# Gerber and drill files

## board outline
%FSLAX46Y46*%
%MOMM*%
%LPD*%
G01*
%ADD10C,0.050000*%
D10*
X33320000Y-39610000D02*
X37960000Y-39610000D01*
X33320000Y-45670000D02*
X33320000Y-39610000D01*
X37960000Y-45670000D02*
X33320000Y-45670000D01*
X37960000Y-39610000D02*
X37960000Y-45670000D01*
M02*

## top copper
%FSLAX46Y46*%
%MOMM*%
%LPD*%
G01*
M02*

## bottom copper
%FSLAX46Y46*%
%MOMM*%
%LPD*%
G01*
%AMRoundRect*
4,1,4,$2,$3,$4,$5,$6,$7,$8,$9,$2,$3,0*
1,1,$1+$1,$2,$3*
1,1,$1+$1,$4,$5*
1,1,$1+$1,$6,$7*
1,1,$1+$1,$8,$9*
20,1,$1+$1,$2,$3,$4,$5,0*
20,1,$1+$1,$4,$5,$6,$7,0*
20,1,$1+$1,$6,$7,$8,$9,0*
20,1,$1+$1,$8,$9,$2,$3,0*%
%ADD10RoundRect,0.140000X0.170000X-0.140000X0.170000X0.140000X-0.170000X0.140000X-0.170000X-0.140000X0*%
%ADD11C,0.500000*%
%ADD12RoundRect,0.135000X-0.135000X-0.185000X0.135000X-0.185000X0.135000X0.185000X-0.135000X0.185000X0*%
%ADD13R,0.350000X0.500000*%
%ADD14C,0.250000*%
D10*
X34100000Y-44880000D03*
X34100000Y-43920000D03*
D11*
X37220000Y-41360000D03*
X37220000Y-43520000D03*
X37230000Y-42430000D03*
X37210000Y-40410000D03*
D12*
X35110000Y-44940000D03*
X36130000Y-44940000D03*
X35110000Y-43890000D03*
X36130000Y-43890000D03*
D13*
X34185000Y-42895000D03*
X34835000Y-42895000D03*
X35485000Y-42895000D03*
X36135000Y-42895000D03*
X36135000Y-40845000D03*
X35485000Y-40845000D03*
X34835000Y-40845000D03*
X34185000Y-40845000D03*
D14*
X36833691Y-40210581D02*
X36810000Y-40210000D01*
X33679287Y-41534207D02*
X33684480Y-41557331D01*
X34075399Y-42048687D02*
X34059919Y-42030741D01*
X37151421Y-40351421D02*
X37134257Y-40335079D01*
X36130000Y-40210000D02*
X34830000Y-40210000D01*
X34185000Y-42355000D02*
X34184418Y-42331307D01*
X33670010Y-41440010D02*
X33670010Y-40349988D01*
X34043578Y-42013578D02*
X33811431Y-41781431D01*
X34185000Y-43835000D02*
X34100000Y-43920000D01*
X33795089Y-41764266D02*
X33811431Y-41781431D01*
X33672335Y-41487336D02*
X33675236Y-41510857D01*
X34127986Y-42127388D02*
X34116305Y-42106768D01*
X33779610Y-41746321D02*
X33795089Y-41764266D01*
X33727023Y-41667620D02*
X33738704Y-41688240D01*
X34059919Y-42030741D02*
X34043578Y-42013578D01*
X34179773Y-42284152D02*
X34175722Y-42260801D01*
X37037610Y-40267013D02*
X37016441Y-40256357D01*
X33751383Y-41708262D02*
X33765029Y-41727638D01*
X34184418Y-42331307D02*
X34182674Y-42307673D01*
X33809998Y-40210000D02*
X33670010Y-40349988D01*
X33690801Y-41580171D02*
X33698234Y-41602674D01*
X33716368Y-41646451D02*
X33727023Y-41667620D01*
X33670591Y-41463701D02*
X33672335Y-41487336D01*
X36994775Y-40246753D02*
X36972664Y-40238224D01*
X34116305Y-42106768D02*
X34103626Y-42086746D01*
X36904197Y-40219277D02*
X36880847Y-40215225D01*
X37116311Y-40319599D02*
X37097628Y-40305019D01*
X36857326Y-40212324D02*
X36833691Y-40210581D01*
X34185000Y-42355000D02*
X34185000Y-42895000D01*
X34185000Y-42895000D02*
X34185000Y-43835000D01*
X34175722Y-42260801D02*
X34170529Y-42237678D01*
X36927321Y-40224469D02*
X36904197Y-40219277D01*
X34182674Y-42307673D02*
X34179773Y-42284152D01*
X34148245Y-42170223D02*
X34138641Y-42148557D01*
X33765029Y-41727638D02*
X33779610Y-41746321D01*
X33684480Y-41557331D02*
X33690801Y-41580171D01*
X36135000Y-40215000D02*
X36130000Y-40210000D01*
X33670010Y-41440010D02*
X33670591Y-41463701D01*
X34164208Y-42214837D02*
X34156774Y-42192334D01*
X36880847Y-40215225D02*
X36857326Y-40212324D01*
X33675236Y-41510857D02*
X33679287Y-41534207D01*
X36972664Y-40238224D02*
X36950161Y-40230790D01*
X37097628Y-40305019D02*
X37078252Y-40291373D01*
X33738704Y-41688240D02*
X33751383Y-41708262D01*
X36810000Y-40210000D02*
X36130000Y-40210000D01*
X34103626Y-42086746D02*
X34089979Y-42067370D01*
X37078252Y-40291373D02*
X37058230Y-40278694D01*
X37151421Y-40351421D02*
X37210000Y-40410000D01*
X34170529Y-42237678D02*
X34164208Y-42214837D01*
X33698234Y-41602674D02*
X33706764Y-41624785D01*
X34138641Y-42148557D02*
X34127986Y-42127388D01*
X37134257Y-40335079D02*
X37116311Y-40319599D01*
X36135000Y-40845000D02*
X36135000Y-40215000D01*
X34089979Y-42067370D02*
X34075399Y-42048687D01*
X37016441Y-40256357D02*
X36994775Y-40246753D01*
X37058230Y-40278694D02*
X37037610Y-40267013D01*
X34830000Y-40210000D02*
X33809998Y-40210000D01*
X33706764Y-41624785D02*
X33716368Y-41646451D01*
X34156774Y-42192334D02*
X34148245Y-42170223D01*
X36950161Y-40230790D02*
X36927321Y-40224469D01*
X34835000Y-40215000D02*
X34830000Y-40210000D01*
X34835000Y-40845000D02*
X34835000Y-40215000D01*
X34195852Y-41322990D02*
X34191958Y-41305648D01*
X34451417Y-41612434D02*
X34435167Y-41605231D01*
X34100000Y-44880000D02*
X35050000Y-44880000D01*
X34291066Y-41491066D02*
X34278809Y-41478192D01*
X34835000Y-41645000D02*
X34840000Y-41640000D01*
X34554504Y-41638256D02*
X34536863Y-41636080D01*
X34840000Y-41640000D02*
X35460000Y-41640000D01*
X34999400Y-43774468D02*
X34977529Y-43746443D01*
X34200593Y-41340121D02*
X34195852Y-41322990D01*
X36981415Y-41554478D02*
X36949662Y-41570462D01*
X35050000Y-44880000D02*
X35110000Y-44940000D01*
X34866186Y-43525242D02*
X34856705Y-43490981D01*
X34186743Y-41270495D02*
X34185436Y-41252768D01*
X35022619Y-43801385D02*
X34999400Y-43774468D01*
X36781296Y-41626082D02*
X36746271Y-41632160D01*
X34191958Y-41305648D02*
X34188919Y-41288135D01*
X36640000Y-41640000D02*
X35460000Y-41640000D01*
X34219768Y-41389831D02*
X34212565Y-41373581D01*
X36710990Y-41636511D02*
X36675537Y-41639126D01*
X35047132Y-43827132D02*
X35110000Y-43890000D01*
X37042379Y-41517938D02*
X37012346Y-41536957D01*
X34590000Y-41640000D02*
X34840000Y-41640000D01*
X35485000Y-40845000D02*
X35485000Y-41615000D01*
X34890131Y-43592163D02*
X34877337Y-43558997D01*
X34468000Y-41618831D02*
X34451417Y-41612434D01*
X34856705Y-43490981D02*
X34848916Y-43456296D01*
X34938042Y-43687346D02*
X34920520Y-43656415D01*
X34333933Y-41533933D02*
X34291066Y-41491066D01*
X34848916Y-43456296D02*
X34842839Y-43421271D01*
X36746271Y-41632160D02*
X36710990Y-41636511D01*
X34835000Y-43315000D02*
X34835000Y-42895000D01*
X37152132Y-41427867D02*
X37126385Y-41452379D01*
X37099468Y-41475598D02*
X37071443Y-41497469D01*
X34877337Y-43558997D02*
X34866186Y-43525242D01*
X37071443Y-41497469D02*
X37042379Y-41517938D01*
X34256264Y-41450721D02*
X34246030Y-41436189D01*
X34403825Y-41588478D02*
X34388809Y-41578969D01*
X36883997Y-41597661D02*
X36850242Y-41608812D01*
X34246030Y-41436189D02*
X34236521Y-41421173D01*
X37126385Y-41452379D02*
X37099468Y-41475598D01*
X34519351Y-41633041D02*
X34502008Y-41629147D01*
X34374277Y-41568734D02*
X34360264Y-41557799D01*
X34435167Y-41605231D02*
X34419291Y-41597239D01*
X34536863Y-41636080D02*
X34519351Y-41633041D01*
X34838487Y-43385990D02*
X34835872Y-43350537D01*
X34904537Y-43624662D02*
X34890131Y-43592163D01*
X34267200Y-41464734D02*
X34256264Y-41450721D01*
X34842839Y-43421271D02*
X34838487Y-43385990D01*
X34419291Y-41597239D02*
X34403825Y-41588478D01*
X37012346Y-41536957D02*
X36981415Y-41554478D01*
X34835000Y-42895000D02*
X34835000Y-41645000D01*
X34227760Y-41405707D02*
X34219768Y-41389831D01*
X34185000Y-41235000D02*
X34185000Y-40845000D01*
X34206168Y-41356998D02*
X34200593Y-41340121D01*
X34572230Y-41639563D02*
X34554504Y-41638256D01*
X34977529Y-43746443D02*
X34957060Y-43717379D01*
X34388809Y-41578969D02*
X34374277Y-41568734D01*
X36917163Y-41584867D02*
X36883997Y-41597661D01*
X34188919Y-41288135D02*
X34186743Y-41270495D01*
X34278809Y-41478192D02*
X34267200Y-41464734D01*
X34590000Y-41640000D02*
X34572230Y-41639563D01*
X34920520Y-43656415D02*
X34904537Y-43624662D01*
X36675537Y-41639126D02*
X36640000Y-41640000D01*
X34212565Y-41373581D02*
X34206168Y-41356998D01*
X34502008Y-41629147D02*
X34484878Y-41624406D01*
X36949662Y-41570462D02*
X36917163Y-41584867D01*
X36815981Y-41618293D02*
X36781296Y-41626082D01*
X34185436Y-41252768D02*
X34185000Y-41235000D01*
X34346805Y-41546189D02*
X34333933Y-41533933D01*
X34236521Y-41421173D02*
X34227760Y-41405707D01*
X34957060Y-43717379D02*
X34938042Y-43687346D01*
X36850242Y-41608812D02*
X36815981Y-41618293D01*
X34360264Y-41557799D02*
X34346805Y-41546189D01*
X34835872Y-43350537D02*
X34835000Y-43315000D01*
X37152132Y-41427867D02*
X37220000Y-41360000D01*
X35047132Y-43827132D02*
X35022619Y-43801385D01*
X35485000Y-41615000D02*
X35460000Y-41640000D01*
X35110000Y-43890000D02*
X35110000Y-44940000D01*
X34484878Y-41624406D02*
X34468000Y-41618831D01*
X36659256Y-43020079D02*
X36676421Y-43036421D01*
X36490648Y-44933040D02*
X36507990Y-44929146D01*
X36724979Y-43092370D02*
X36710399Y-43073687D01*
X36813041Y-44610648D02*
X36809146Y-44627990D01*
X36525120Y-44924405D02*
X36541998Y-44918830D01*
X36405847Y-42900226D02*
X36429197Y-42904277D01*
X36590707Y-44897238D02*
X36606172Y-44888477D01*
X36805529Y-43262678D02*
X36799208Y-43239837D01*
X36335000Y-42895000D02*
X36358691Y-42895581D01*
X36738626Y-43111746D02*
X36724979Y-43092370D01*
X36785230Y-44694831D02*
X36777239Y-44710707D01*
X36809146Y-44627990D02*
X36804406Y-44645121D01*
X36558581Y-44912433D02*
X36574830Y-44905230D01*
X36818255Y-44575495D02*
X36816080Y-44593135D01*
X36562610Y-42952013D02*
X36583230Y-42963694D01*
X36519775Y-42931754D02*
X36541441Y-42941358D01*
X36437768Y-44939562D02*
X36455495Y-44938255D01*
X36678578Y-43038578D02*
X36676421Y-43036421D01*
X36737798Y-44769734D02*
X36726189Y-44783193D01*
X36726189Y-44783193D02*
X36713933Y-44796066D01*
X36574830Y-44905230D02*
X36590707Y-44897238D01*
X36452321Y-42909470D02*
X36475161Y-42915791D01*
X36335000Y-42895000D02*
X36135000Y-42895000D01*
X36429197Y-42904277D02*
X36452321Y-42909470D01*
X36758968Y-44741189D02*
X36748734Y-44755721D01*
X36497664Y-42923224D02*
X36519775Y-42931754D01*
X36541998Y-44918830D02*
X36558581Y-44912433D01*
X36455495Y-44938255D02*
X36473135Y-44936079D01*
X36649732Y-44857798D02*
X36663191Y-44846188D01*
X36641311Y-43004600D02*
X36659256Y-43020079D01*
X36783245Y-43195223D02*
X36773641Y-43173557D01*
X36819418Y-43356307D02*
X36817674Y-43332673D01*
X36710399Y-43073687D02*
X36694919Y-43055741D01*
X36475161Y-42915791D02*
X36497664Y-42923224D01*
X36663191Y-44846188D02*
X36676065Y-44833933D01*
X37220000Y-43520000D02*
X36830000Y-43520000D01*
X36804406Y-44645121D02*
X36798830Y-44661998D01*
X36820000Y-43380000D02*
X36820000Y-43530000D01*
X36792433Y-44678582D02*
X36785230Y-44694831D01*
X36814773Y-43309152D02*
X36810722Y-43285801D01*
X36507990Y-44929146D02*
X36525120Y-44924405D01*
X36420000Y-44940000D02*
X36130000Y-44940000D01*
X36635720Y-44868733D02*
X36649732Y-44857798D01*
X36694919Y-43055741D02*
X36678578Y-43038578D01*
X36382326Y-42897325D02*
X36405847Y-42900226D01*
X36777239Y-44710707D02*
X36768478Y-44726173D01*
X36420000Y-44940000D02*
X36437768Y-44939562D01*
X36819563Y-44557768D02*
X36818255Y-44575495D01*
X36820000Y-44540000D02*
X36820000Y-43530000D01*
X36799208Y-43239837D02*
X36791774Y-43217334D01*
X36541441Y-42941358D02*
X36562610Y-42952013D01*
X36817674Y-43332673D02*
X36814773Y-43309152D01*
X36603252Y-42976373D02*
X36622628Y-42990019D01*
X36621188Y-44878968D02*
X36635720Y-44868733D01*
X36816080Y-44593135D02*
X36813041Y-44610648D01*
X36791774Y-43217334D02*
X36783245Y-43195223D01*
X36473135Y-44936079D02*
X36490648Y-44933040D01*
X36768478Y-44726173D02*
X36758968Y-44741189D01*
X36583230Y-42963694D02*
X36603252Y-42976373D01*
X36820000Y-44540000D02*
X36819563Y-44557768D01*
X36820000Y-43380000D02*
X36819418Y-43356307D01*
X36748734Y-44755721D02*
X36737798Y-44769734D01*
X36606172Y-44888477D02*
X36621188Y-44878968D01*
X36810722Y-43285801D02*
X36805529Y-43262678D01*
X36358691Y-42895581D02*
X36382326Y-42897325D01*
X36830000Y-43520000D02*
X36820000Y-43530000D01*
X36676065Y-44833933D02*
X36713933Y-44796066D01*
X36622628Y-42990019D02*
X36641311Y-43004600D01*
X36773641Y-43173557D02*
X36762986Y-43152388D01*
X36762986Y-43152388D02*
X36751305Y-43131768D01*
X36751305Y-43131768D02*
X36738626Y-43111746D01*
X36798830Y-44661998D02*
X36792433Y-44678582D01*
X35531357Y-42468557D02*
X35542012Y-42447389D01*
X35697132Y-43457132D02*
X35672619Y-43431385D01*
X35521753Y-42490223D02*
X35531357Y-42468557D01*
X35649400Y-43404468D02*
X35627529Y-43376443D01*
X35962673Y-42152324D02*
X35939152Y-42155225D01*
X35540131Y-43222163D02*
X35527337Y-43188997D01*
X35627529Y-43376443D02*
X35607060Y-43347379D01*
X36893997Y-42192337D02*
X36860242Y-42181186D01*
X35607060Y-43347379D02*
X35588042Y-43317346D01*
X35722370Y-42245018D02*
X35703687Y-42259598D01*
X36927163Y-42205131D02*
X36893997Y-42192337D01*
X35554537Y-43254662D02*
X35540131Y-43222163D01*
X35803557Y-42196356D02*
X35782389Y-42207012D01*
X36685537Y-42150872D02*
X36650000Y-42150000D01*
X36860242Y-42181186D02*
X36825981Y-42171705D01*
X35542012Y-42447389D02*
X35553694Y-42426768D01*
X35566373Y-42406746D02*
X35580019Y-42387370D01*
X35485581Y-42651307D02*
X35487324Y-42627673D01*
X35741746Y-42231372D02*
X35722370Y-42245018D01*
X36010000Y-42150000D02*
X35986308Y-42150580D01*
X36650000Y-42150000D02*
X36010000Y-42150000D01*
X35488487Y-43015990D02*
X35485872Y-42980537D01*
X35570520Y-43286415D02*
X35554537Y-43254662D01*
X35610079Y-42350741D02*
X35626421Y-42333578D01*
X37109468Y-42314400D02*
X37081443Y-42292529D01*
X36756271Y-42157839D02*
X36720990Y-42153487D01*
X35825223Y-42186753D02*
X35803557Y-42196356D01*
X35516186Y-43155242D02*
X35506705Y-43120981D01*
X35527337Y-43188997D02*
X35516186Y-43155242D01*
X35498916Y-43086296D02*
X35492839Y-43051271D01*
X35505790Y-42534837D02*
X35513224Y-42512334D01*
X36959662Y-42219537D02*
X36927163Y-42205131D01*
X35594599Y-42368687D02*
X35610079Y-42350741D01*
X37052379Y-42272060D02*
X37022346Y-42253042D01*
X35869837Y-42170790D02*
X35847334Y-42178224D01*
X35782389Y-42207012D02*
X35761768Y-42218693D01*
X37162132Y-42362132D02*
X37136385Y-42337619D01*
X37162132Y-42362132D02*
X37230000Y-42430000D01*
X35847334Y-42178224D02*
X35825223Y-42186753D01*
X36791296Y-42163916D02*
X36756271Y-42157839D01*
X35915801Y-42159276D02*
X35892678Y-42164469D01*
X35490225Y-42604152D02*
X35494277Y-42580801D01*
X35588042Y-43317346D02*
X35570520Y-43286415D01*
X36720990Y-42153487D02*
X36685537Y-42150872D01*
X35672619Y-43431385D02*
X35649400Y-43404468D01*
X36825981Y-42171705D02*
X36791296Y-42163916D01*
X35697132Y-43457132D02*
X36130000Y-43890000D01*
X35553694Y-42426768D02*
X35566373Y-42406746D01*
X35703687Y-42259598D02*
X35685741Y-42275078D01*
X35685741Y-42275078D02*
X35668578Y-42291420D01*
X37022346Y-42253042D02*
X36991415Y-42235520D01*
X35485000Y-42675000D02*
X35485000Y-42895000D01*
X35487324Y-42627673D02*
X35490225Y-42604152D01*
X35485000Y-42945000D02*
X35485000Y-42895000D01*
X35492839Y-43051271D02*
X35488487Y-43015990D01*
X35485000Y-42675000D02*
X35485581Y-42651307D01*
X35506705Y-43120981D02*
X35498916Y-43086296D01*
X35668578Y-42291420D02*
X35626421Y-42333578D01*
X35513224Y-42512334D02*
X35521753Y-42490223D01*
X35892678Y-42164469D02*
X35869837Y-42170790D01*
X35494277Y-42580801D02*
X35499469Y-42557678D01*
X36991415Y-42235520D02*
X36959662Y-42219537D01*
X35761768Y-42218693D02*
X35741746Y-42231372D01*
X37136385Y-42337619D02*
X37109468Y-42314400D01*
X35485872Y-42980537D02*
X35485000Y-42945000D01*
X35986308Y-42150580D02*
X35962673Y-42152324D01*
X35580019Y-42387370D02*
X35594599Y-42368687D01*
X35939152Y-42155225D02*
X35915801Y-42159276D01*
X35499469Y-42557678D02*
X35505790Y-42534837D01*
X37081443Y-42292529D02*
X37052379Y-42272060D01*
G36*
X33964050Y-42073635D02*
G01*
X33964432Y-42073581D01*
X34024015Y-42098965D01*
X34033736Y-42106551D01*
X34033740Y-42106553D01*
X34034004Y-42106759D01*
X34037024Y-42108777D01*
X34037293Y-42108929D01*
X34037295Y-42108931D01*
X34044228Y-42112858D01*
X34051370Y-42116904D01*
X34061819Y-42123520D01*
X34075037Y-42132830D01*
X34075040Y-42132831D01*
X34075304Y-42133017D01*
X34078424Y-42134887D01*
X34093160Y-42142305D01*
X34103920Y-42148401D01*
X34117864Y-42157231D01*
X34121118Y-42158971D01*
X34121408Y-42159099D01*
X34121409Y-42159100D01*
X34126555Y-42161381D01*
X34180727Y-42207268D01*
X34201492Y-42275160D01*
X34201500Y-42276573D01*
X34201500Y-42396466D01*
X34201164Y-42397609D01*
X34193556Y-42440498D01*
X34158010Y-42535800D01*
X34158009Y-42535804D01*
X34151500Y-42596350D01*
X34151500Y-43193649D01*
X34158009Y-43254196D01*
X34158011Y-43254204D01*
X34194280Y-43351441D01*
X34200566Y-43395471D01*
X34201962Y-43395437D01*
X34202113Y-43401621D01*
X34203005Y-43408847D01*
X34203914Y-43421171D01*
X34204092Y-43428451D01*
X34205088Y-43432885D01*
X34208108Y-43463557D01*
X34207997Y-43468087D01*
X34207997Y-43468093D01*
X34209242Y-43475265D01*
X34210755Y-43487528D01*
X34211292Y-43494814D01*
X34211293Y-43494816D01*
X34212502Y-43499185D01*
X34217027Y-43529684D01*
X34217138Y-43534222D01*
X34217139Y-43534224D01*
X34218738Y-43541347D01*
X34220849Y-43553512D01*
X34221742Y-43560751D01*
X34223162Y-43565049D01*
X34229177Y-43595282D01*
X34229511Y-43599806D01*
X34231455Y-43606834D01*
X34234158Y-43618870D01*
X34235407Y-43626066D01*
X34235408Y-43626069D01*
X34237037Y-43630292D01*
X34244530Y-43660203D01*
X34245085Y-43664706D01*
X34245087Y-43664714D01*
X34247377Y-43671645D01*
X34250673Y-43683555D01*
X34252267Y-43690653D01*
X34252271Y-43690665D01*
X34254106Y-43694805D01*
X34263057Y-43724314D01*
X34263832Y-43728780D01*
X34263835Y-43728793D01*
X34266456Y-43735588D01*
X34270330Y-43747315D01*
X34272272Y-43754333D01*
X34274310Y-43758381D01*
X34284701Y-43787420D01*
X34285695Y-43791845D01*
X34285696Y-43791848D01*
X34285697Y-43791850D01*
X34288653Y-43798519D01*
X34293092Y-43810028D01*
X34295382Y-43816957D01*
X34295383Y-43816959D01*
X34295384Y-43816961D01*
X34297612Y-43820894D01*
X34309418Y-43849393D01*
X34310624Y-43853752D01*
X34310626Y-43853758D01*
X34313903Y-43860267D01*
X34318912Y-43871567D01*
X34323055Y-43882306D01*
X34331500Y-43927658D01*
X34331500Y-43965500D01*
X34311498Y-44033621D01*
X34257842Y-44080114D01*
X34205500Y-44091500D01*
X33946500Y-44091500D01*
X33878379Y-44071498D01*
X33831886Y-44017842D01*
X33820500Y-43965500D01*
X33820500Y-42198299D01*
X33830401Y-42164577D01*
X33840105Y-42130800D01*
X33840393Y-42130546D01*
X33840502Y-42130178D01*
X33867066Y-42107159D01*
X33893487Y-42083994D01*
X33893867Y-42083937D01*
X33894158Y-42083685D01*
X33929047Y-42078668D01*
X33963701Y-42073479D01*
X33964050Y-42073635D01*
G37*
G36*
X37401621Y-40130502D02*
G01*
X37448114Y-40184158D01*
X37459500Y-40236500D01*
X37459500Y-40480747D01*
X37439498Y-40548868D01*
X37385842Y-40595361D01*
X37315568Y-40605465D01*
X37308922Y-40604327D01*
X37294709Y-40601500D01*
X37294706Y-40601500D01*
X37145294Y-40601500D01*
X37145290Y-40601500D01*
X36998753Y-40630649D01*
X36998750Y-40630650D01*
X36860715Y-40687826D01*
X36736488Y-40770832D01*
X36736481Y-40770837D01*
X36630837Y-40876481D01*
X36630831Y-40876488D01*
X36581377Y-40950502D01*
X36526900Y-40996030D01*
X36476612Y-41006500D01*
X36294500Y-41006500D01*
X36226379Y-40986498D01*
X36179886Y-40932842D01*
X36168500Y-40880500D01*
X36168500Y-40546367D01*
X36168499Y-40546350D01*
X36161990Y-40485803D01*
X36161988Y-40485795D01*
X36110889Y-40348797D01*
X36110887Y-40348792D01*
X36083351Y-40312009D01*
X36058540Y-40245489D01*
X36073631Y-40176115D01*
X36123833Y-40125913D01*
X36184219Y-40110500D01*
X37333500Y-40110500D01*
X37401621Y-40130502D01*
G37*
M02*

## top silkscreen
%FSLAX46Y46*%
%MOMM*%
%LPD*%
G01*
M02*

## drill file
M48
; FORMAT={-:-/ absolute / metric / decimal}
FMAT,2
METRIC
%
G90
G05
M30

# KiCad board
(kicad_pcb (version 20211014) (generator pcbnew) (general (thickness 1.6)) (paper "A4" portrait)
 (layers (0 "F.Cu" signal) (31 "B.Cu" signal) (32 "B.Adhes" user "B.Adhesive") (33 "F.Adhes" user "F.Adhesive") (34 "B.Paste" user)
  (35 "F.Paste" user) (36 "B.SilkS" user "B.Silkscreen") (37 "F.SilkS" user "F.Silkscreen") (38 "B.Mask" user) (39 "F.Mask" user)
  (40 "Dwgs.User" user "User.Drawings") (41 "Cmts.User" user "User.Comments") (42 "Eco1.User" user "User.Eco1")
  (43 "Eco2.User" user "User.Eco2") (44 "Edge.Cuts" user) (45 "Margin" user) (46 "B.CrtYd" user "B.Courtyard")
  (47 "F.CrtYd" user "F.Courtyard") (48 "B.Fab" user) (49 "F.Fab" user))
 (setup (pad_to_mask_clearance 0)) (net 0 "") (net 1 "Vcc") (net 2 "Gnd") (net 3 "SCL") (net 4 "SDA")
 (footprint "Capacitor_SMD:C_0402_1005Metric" (layer "B.Cu") (at 34.1 44.4 90)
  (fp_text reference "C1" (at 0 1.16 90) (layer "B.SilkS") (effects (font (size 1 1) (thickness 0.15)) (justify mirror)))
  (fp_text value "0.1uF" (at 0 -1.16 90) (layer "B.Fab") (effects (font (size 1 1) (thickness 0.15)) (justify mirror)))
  (pad "1" smd roundrect locked (at -0.48 0 90) (size 0.56 0.62) (layers "B.Cu" "B.Paste" "B.Mask") (roundrect_rratio 0.25) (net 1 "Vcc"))
  (pad "2" smd roundrect locked (at 0.48 0 90) (size 0.56 0.62) (layers "B.Cu" "B.Paste" "B.Mask") (roundrect_rratio 0.25) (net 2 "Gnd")))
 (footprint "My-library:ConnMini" (layer "B.Cu") (at 37.22 41.36)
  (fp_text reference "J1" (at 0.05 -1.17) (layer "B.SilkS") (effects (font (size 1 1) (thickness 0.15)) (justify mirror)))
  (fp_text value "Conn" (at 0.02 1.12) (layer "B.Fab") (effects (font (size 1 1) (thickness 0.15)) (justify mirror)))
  (pad "1" smd circle locked (at 0 0) (size 0.5 0.5) (layers "B.Cu" "B.Paste" "B.Mask") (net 1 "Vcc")))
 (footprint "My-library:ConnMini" (layer "B.Cu") (at 37.22 43.52)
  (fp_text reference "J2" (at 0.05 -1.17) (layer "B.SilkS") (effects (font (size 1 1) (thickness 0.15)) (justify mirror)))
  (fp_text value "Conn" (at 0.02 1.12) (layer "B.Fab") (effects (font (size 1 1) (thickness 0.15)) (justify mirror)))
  (pad "1" smd circle locked (at 0 0) (size 0.5 0.5) (layers "B.Cu" "B.Paste" "B.Mask") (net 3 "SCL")))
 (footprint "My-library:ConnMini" (layer "B.Cu") (at 37.23 42.43)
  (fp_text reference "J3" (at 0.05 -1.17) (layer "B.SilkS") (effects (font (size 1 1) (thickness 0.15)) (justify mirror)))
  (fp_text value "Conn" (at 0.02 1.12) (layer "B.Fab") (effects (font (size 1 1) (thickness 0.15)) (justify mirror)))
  (pad "1" smd circle locked (at 0 0) (size 0.5 0.5) (layers "B.Cu" "B.Paste" "B.Mask") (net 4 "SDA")))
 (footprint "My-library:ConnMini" (layer "B.Cu") (at 37.21 40.41)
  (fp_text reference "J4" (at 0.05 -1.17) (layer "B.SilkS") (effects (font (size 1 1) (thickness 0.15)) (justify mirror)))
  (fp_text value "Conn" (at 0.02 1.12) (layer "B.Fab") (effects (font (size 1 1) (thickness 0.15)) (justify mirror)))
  (pad "1" smd circle locked (at 0 0) (size 0.5 0.5) (layers "B.Cu" "B.Paste" "B.Mask") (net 2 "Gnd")))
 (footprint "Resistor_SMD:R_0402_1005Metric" (layer "B.Cu") (at 35.62 44.94)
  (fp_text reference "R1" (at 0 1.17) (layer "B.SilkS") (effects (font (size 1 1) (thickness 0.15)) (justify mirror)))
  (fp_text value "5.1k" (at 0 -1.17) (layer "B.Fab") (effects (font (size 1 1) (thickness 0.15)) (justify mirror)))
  (pad "1" smd roundrect locked (at -0.51 0) (size 0.54 0.64) (layers "B.Cu" "B.Paste" "B.Mask") (roundrect_rratio 0.25) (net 1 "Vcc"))
  (pad "2" smd roundrect locked (at 0.51 0) (size 0.54 0.64) (layers "B.Cu" "B.Paste" "B.Mask") (roundrect_rratio 0.25) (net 3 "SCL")))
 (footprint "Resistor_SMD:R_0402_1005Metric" (layer "B.Cu") (at 35.62 43.89)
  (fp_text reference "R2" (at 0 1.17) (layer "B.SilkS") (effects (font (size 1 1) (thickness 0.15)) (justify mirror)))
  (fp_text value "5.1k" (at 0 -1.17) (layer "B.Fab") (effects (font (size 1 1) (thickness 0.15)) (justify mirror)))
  (pad "1" smd roundrect locked (at -0.51 0) (size 0.54 0.64) (layers "B.Cu" "B.Paste" "B.Mask") (roundrect_rratio 0.25) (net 1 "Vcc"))
  (pad "2" smd roundrect locked (at 0.51 0) (size 0.54 0.64) (layers "B.Cu" "B.Paste" "B.Mask") (roundrect_rratio 0.25) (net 4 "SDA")))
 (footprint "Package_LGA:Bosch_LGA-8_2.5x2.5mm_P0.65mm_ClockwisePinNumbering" (layer "B.Cu") (at 35.16 41.87)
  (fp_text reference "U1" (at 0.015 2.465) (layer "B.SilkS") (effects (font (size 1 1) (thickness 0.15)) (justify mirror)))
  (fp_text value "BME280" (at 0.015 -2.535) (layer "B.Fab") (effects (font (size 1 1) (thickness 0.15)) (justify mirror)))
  (pad "1" smd rect locked (at -0.975 1.025 270) (size 0.5 0.35) (layers "B.Cu" "B.Paste" "B.Mask") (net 2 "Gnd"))
  (pad "2" smd rect locked (at -0.325 1.025 270) (size 0.5 0.35) (layers "B.Cu" "B.Paste" "B.Mask") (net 1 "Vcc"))
  (pad "3" smd rect locked (at 0.325 1.025 270) (size 0.5 0.35) (layers "B.Cu" "B.Paste" "B.Mask") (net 4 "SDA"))
  (pad "4" smd rect locked (at 0.975 1.025 270) (size 0.5 0.35) (layers "B.Cu" "B.Paste" "B.Mask") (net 3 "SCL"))
  (pad "5" smd rect locked (at 0.975 -1.025 270) (size 0.5 0.35) (layers "B.Cu" "B.Paste" "B.Mask") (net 2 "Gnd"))
  (pad "6" smd rect locked (at 0.325 -1.025 270) (size 0.5 0.35) (layers "B.Cu" "B.Paste" "B.Mask") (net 1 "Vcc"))
  (pad "7" smd rect locked (at -0.325 -1.025 270) (size 0.5 0.35) (layers "B.Cu" "B.Paste" "B.Mask") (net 2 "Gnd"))
  (pad "8" smd rect locked (at -0.975 -1.025 270) (size 0.5 0.35) (layers "B.Cu" "B.Paste" "B.Mask") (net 1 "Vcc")))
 (gr_line (start 33.32 39.61) (end 37.96 39.61) (layer "Edge.Cuts") (width 0.05))
 (gr_line (start 33.32 45.67) (end 33.32 39.61) (layer "Edge.Cuts") (width 0.05))
 (gr_line (start 37.96 45.67) (end 33.32 45.67) (layer "Edge.Cuts") (width 0.05))
 (gr_line (start 37.96 39.61) (end 37.96 45.67) (layer "Edge.Cuts") (width 0.05))
 (segment (start 36.833691 40.210581) (end 36.81 40.21) (width 0.25) (layer "B.Cu") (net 2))
 (segment (start 33.679287 41.534207) (end 33.68448 41.557331) (width 0.25) (layer "B.Cu") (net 2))
 (segment (start 34.075399 42.048687) (end 34.059919 42.030741) (width 0.25) (layer "B.Cu") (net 2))
 (segment (start 37.151421 40.351421) (end 37.134257 40.335079) (width 0.25) (layer "B.Cu") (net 2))
 (segment (start 36.13 40.21) (end 34.83 40.21) (width 0.25) (layer "B.Cu") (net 2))
 (segment (start 34.185 42.355) (end 34.184418 42.331307) (width 0.25) (layer "B.Cu") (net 2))
 (segment (start 33.67001 41.44001) (end 33.67001 40.349988) (width 0.25) (layer "B.Cu") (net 2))
 (segment (start 34.043578 42.013578) (end 33.811431 41.781431) (width 0.25) (layer "B.Cu") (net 2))
 (segment (start 34.185 43.835) (end 34.1 43.92) (width 0.25) (layer "B.Cu") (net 2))
 (segment (start 33.795089 41.764266) (end 33.811431 41.781431) (width 0.25) (layer "B.Cu") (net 2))
 (segment (start 33.672335 41.487336) (end 33.675236 41.510857) (width 0.25) (layer "B.Cu") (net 2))
 (segment (start 34.127986 42.127388) (end 34.116305 42.106768) (width 0.25) (layer "B.Cu") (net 2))
 (segment (start 33.77961 41.746321) (end 33.795089 41.764266) (width 0.25) (layer "B.Cu") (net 2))
 (segment (start 33.727023 41.66762) (end 33.738704 41.68824) (width 0.25) (layer "B.Cu") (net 2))
 (segment (start 34.059919 42.030741) (end 34.043578 42.013578) (width 0.25) (layer "B.Cu") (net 2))
 (segment (start 34.179773 42.284152) (end 34.175722 42.260801) (width 0.25) (layer "B.Cu") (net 2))
 (segment (start 37.03761 40.267013) (end 37.016441 40.256357) (width 0.25) (layer "B.Cu") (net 2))
 (segment (start 33.751383 41.708262) (end 33.765029 41.727638) (width 0.25) (layer "B.Cu") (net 2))
 (segment (start 34.184418 42.331307) (end 34.182674 42.307673) (width 0.25) (layer "B.Cu") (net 2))
 (segment (start 33.809998 40.21) (end 33.67001 40.349988) (width 0.25) (layer "B.Cu") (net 2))
 (segment (start 33.690801 41.580171) (end 33.698234 41.602674) (width 0.25) (layer "B.Cu") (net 2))
 (segment (start 33.716368 41.646451) (end 33.727023 41.66762) (width 0.25) (layer "B.Cu") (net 2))
 (segment (start 33.670591 41.463701) (end 33.672335 41.487336) (width 0.25) (layer "B.Cu") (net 2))
 (segment (start 36.994775 40.246753) (end 36.972664 40.238224) (width 0.25) (layer "B.Cu") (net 2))
 (segment (start 34.116305 42.106768) (end 34.103626 42.086746) (width 0.25) (layer "B.Cu") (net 2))
 (segment (start 36.904197 40.219277) (end 36.880847 40.215225) (width 0.25) (layer "B.Cu") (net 2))
 (segment (start 37.116311 40.319599) (end 37.097628 40.305019) (width 0.25) (layer "B.Cu") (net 2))
 (segment (start 36.857326 40.212324) (end 36.833691 40.210581) (width 0.25) (layer "B.Cu") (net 2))
 (segment (start 34.185 42.355) (end 34.185 42.895) (width 0.25) (layer "B.Cu") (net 2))
 (segment (start 34.185 42.895) (end 34.185 43.835) (width 0.25) (layer "B.Cu") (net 2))
 (segment (start 34.175722 42.260801) (end 34.170529 42.237678) (width 0.25) (layer "B.Cu") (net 2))
 (segment (start 36.927321 40.224469) (end 36.904197 40.219277) (width 0.25) (layer "B.Cu") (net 2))
 (segment (start 34.182674 42.307673) (end 34.179773 42.284152) (width 0.25) (layer "B.Cu") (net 2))
 (segment (start 34.148245 42.170223) (end 34.138641 42.148557) (width 0.25) (layer "B.Cu") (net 2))
 (segment (start 33.765029 41.727638) (end 33.77961 41.746321) (width 0.25) (layer "B.Cu") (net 2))
 (segment (start 33.68448 41.557331) (end 33.690801 41.580171) (width 0.25) (layer "B.Cu") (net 2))
 (segment (start 36.135 40.215) (end 36.13 40.21) (width 0.25) (layer "B.Cu") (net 2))
 (segment (start 33.67001 41.44001) (end 33.670591 41.463701) (width 0.25) (layer "B.Cu") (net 2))
 (segment (start 34.164208 42.214837) (end 34.156774 42.192334) (width 0.25) (layer "B.Cu") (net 2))
 (segment (start 36.880847 40.215225) (end 36.857326 40.212324) (width 0.25) (layer "B.Cu") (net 2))
 (segment (start 33.675236 41.510857) (end 33.679287 41.534207) (width 0.25) (layer "B.Cu") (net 2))
 (segment (start 36.972664 40.238224) (end 36.950161 40.23079) (width 0.25) (layer "B.Cu") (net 2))
 (segment (start 37.097628 40.305019) (end 37.078252 40.291373) (width 0.25) (layer "B.Cu") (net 2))
 (segment (start 33.738704 41.68824) (end 33.751383 41.708262) (width 0.25) (layer "B.Cu") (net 2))
 (segment (start 36.81 40.21) (end 36.13 40.21) (width 0.25) (layer "B.Cu") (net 2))
 (segment (start 34.103626 42.086746) (end 34.089979 42.06737) (width 0.25) (layer "B.Cu") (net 2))
 (segment (start 37.078252 40.291373) (end 37.05823 40.278694) (width 0.25) (layer "B.Cu") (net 2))
 (segment (start 37.151421 40.351421) (end 37.21 40.41) (width 0.25) (layer "B.Cu") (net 2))
 (segment (start 34.170529 42.237678) (end 34.164208 42.214837) (width 0.25) (layer "B.Cu") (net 2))
 (segment (start 33.698234 41.602674) (end 33.706764 41.624785) (width 0.25) (layer "B.Cu") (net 2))
 (segment (start 34.138641 42.148557) (end 34.127986 42.127388) (width 0.25) (layer "B.Cu") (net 2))
 (segment (start 37.134257 40.335079) (end 37.116311 40.319599) (width 0.25) (layer "B.Cu") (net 2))
 (segment (start 36.135 40.845) (end 36.135 40.215) (width 0.25) (layer "B.Cu") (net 2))
 (segment (start 34.089979 42.06737) (end 34.075399 42.048687) (width 0.25) (layer "B.Cu") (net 2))
 (segment (start 37.016441 40.256357) (end 36.994775 40.246753) (width 0.25) (layer "B.Cu") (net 2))
 (segment (start 37.05823 40.278694) (end 37.03761 40.267013) (width 0.25) (layer "B.Cu") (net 2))
 (segment (start 34.83 40.21) (end 33.809998 40.21) (width 0.25) (layer "B.Cu") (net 2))
 (segment (start 33.706764 41.624785) (end 33.716368 41.646451) (width 0.25) (layer "B.Cu") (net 2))
 (segment (start 34.156774 42.192334) (end 34.148245 42.170223) (width 0.25) (layer "B.Cu") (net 2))
 (segment (start 36.950161 40.23079) (end 36.927321 40.224469) (width 0.25) (layer "B.Cu") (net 2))
 (segment (start 34.835 40.215) (end 34.83 40.21) (width 0.25) (layer "B.Cu") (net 2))
 (segment (start 34.835 40.845) (end 34.835 40.215) (width 0.25) (layer "B.Cu") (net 2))
 (segment (start 34.195852 41.32299) (end 34.191958 41.305648) (width 0.25) (layer "B.Cu") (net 1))
 (segment (start 34.451417 41.612434) (end 34.435167 41.605231) (width 0.25) (layer "B.Cu") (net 1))
 (segment (start 34.1 44.88) (end 35.05 44.88) (width 0.25) (layer "B.Cu") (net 1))
 (segment (start 34.291066 41.491066) (end 34.278809 41.478192) (width 0.25) (layer "B.Cu") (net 1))
 (segment (start 34.835 41.645) (end 34.84 41.64) (width 0.25) (layer "B.Cu") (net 1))
 (segment (start 34.554504 41.638256) (end 34.536863 41.63608) (width 0.25) (layer "B.Cu") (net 1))
 (segment (start 34.84 41.64) (end 35.46 41.64) (width 0.25) (layer "B.Cu") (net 1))
 (segment (start 34.9994 43.774468) (end 34.977529 43.746443) (width 0.25) (layer "B.Cu") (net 1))
 (segment (start 34.200593 41.340121) (end 34.195852 41.32299) (width 0.25) (layer "B.Cu") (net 1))
 (segment (start 36.981415 41.554478) (end 36.949662 41.570462) (width 0.25) (layer "B.Cu") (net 1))
 (segment (start 35.05 44.88) (end 35.11 44.94) (width 0.25) (layer "B.Cu") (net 1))
 (segment (start 34.866186 43.525242) (end 34.856705 43.490981) (width 0.25) (layer "B.Cu") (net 1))
 (segment (start 34.186743 41.270495) (end 34.185436 41.252768) (width 0.25) (layer "B.Cu") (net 1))
 (segment (start 35.022619 43.801385) (end 34.9994 43.774468) (width 0.25) (layer "B.Cu") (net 1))
 (segment (start 36.781296 41.626082) (end 36.746271 41.63216) (width 0.25) (layer "B.Cu") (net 1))
 (segment (start 34.191958 41.305648) (end 34.188919 41.288135) (width 0.25) (layer "B.Cu") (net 1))
 (segment (start 36.64 41.64) (end 35.46 41.64) (width 0.25) (layer "B.Cu") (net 1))
 (segment (start 34.219768 41.389831) (end 34.212565 41.373581) (width 0.25) (layer "B.Cu") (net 1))
 (segment (start 36.71099 41.636511) (end 36.675537 41.639126) (width 0.25) (layer "B.Cu") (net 1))
 (segment (start 35.047132 43.827132) (end 35.11 43.89) (width 0.25) (layer "B.Cu") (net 1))
 (segment (start 37.042379 41.517938) (end 37.012346 41.536957) (width 0.25) (layer "B.Cu") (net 1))
 (segment (start 34.59 41.64) (end 34.84 41.64) (width 0.25) (layer "B.Cu") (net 1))
 (segment (start 35.485 40.845) (end 35.485 41.615) (width 0.25) (layer "B.Cu") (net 1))
 (segment (start 34.890131 43.592163) (end 34.877337 43.558997) (width 0.25) (layer "B.Cu") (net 1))
 (segment (start 34.468 41.618831) (end 34.451417 41.612434) (width 0.25) (layer "B.Cu") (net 1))
 (segment (start 34.856705 43.490981) (end 34.848916 43.456296) (width 0.25) (layer "B.Cu") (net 1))
 (segment (start 34.938042 43.687346) (end 34.92052 43.656415) (width 0.25) (layer "B.Cu") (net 1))
 (segment (start 34.333933 41.533933) (end 34.291066 41.491066) (width 0.25) (layer "B.Cu") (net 1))
 (segment (start 34.848916 43.456296) (end 34.842839 43.421271) (width 0.25) (layer "B.Cu") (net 1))
 (segment (start 36.746271 41.63216) (end 36.71099 41.636511) (width 0.25) (layer "B.Cu") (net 1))
 (segment (start 34.835 43.315) (end 34.835 42.895) (width 0.25) (layer "B.Cu") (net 1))
 (segment (start 37.152132 41.427867) (end 37.126385 41.452379) (width 0.25) (layer "B.Cu") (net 1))
 (segment (start 37.099468 41.475598) (end 37.071443 41.497469) (width 0.25) (layer "B.Cu") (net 1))
 (segment (start 34.877337 43.558997) (end 34.866186 43.525242) (width 0.25) (layer "B.Cu") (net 1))
 (segment (start 37.071443 41.497469) (end 37.042379 41.517938) (width 0.25) (layer "B.Cu") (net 1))
 (segment (start 34.256264 41.450721) (end 34.24603 41.436189) (width 0.25) (layer "B.Cu") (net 1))
 (segment (start 34.403825 41.588478) (end 34.388809 41.578969) (width 0.25) (layer "B.Cu") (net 1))
 (segment (start 36.883997 41.597661) (end 36.850242 41.608812) (width 0.25) (layer "B.Cu") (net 1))
 (segment (start 34.24603 41.436189) (end 34.236521 41.421173) (width 0.25) (layer "B.Cu") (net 1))
 (segment (start 37.126385 41.452379) (end 37.099468 41.475598) (width 0.25) (layer "B.Cu") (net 1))
 (segment (start 34.519351 41.633041) (end 34.502008 41.629147) (width 0.25) (layer "B.Cu") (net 1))
 (segment (start 34.374277 41.568734) (end 34.360264 41.557799) (width 0.25) (layer "B.Cu") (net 1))
 (segment (start 34.435167 41.605231) (end 34.419291 41.597239) (width 0.25) (layer "B.Cu") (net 1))
 (segment (start 34.536863 41.63608) (end 34.519351 41.633041) (width 0.25) (layer "B.Cu") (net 1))
 (segment (start 34.838487 43.38599) (end 34.835872 43.350537) (width 0.25) (layer "B.Cu") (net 1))
 (segment (start 34.904537 43.624662) (end 34.890131 43.592163) (width 0.25) (layer "B.Cu") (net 1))
 (segment (start 34.2672 41.464734) (end 34.256264 41.450721) (width 0.25) (layer "B.Cu") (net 1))
 (segment (start 34.842839 43.421271) (end 34.838487 43.38599) (width 0.25) (layer "B.Cu") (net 1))
 (segment (start 34.419291 41.597239) (end 34.403825 41.588478) (width 0.25) (layer "B.Cu") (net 1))
 (segment (start 37.012346 41.536957) (end 36.981415 41.554478) (width 0.25) (layer "B.Cu") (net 1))
 (segment (start 34.835 42.895) (end 34.835 41.645) (width 0.25) (layer "B.Cu") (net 1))
 (segment (start 34.22776 41.405707) (end 34.219768 41.389831) (width 0.25) (layer "B.Cu") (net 1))
 (segment (start 34.185 41.235) (end 34.185 40.845) (width 0.25) (layer "B.Cu") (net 1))
 (segment (start 34.206168 41.356998) (end 34.200593 41.340121) (width 0.25) (layer "B.Cu") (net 1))
 (segment (start 34.57223 41.639563) (end 34.554504 41.638256) (width 0.25) (layer "B.Cu") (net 1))
 (segment (start 34.977529 43.746443) (end 34.95706 43.717379) (width 0.25) (layer "B.Cu") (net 1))
 (segment (start 34.388809 41.578969) (end 34.374277 41.568734) (width 0.25) (layer "B.Cu") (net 1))
 (segment (start 36.917163 41.584867) (end 36.883997 41.597661) (width 0.25) (layer "B.Cu") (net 1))
 (segment (start 34.188919 41.288135) (end 34.186743 41.270495) (width 0.25) (layer "B.Cu") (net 1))
 (segment (start 34.278809 41.478192) (end 34.2672 41.464734) (width 0.25) (layer "B.Cu") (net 1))
 (segment (start 34.59 41.64) (end 34.57223 41.639563) (width 0.25) (layer "B.Cu") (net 1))
 (segment (start 34.92052 43.656415) (end 34.904537 43.624662) (width 0.25) (layer "B.Cu") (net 1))
 (segment (start 36.675537 41.639126) (end 36.64 41.64) (width 0.25) (layer "B.Cu") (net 1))
 (segment (start 34.212565 41.373581) (end 34.206168 41.356998) (width 0.25) (layer "B.Cu") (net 1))
 (segment (start 34.502008 41.629147) (end 34.484878 41.624406) (width 0.25) (layer "B.Cu") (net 1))
 (segment (start 36.949662 41.570462) (end 36.917163 41.584867) (width 0.25) (layer "B.Cu") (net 1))
 (segment (start 36.815981 41.618293) (end 36.781296 41.626082) (width 0.25) (layer "B.Cu") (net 1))
 (segment (start 34.185436 41.252768) (end 34.185 41.235) (width 0.25) (layer "B.Cu") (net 1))
 (segment (start 34.346805 41.546189) (end 34.333933 41.533933) (width 0.25) (layer "B.Cu") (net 1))
 (segment (start 34.236521 41.421173) (end 34.22776 41.405707) (width 0.25) (layer "B.Cu") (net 1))
 (segment (start 34.95706 43.717379) (end 34.938042 43.687346) (width 0.25) (layer "B.Cu") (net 1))
 (segment (start 36.850242 41.608812) (end 36.815981 41.618293) (width 0.25) (layer "B.Cu") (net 1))
 (segment (start 34.360264 41.557799) (end 34.346805 41.546189) (width 0.25) (layer "B.Cu") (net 1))
 (segment (start 34.835872 43.350537) (end 34.835 43.315) (width 0.25) (layer "B.Cu") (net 1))
 (segment (start 37.152132 41.427867) (end 37.22 41.36) (width 0.25) (layer "B.Cu") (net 1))
 (segment (start 35.047132 43.827132) (end 35.022619 43.801385) (width 0.25) (layer "B.Cu") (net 1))
 (segment (start 35.485 41.615) (end 35.46 41.64) (width 0.25) (layer "B.Cu") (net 1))
 (segment (start 35.11 43.89) (end 35.11 44.94) (width 0.25) (layer "B.Cu") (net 1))
 (segment (start 34.484878 41.624406) (end 34.468 41.618831) (width 0.25) (layer "B.Cu") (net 1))
 (segment (start 36.659256 43.020079) (end 36.676421 43.036421) (width 0.25) (layer "B.Cu") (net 3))
 (segment (start 36.490648 44.93304) (end 36.50799 44.929146) (width 0.25) (layer "B.Cu") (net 3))
 (segment (start 36.724979 43.09237) (end 36.710399 43.073687) (width 0.25) (layer "B.Cu") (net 3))
 (segment (start 36.813041 44.610648) (end 36.809146 44.62799) (width 0.25) (layer "B.Cu") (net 3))
 (segment (start 36.52512 44.924405) (end 36.541998 44.91883) (width 0.25) (layer "B.Cu") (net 3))
 (segment (start 36.405847 42.900226) (end 36.429197 42.904277) (width 0.25) (layer "B.Cu") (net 3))
 (segment (start 36.590707 44.897238) (end 36.606172 44.888477) (width 0.25) (layer "B.Cu") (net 3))
 (segment (start 36.805529 43.262678) (end 36.799208 43.239837) (width 0.25) (layer "B.Cu") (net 3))
 (segment (start 36.335 42.895) (end 36.358691 42.895581) (width 0.25) (layer "B.Cu") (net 3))
 (segment (start 36.738626 43.111746) (end 36.724979 43.09237) (width 0.25) (layer "B.Cu") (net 3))
 (segment (start 36.78523 44.694831) (end 36.777239 44.710707) (width 0.25) (layer "B.Cu") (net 3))
 (segment (start 36.809146 44.62799) (end 36.804406 44.645121) (width 0.25) (layer "B.Cu") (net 3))
 (segment (start 36.558581 44.912433) (end 36.57483 44.90523) (width 0.25) (layer "B.Cu") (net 3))
 (segment (start 36.818255 44.575495) (end 36.81608 44.593135) (width 0.25) (layer "B.Cu") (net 3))
 (segment (start 36.56261 42.952013) (end 36.58323 42.963694) (width 0.25) (layer "B.Cu") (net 3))
 (segment (start 36.519775 42.931754) (end 36.541441 42.941358) (width 0.25) (layer "B.Cu") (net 3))
 (segment (start 36.437768 44.939562) (end 36.455495 44.938255) (width 0.25) (layer "B.Cu") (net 3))
 (segment (start 36.678578 43.038578) (end 36.676421 43.036421) (width 0.25) (layer "B.Cu") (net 3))
 (segment (start 36.737798 44.769734) (end 36.726189 44.783193) (width 0.25) (layer "B.Cu") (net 3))
 (segment (start 36.726189 44.783193) (end 36.713933 44.796066) (width 0.25) (layer "B.Cu") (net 3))
 (segment (start 36.57483 44.90523) (end 36.590707 44.897238) (width 0.25) (layer "B.Cu") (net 3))
 (segment (start 36.452321 42.90947) (end 36.475161 42.915791) (width 0.25) (layer "B.Cu") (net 3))
 (segment (start 36.335 42.895) (end 36.135 42.895) (width 0.25) (layer "B.Cu") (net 3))
 (segment (start 36.429197 42.904277) (end 36.452321 42.90947) (width 0.25) (layer "B.Cu") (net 3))
 (segment (start 36.758968 44.741189) (end 36.748734 44.755721) (width 0.25) (layer "B.Cu") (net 3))
 (segment (start 36.497664 42.923224) (end 36.519775 42.931754) (width 0.25) (layer "B.Cu") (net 3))
 (segment (start 36.541998 44.91883) (end 36.558581 44.912433) (width 0.25) (layer "B.Cu") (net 3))
 (segment (start 36.455495 44.938255) (end 36.473135 44.936079) (width 0.25) (layer "B.Cu") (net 3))
 (segment (start 36.649732 44.857798) (end 36.663191 44.846188) (width 0.25) (layer "B.Cu") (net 3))
 (segment (start 36.641311 43.0046) (end 36.659256 43.020079) (width 0.25) (layer "B.Cu") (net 3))
 (segment (start 36.783245 43.195223) (end 36.773641 43.173557) (width 0.25) (layer "B.Cu") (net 3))
 (segment (start 36.819418 43.356307) (end 36.817674 43.332673) (width 0.25) (layer "B.Cu") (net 3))
 (segment (start 36.710399 43.073687) (end 36.694919 43.055741) (width 0.25) (layer "B.Cu") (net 3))
 (segment (start 36.475161 42.915791) (end 36.497664 42.923224) (width 0.25) (layer "B.Cu") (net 3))
 (segment (start 36.663191 44.846188) (end 36.676065 44.833933) (width 0.25) (layer "B.Cu") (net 3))
 (segment (start 37.22 43.52) (end 36.83 43.52) (width 0.25) (layer "B.Cu") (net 3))
 (segment (start 36.804406 44.645121) (end 36.79883 44.661998) (width 0.25) (layer "B.Cu") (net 3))
 (segment (start 36.82 43.38) (end 36.82 43.53) (width 0.25) (layer "B.Cu") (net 3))
 (segment (start 36.792433 44.678582) (end 36.78523 44.694831) (width 0.25) (layer "B.Cu") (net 3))
 (segment (start 36.814773 43.309152) (end 36.810722 43.285801) (width 0.25) (layer "B.Cu") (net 3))
 (segment (start 36.50799 44.929146) (end 36.52512 44.924405) (width 0.25) (layer "B.Cu") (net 3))
 (segment (start 36.42 44.94) (end 36.13 44.94) (width 0.25) (layer "B.Cu") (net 3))
 (segment (start 36.63572 44.868733) (end 36.649732 44.857798) (width 0.25) (layer "B.Cu") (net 3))
 (segment (start 36.694919 43.055741) (end 36.678578 43.038578) (width 0.25) (layer "B.Cu") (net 3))
 (segment (start 36.382326 42.897325) (end 36.405847 42.900226) (width 0.25) (layer "B.Cu") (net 3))
 (segment (start 36.777239 44.710707) (end 36.768478 44.726173) (width 0.25) (layer "B.Cu") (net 3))
 (segment (start 36.42 44.94) (end 36.437768 44.939562) (width 0.25) (layer "B.Cu") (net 3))
 (segment (start 36.819563 44.557768) (end 36.818255 44.575495) (width 0.25) (layer "B.Cu") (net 3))
 (segment (start 36.82 44.54) (end 36.82 43.53) (width 0.25) (layer "B.Cu") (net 3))
 (segment (start 36.799208 43.239837) (end 36.791774 43.217334) (width 0.25) (layer "B.Cu") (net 3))
 (segment (start 36.541441 42.941358) (end 36.56261 42.952013) (width 0.25) (layer "B.Cu") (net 3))
 (segment (start 36.817674 43.332673) (end 36.814773 43.309152) (width 0.25) (layer "B.Cu") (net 3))
 (segment (start 36.603252 42.976373) (end 36.622628 42.990019) (width 0.25) (layer "B.Cu") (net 3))
 (segment (start 36.621188 44.878968) (end 36.63572 44.868733) (width 0.25) (layer "B.Cu") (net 3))
 (segment (start 36.81608 44.593135) (end 36.813041 44.610648) (width 0.25) (layer "B.Cu") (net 3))
 (segment (start 36.791774 43.217334) (end 36.783245 43.195223) (width 0.25) (layer "B.Cu") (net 3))
 (segment (start 36.473135 44.936079) (end 36.490648 44.93304) (width 0.25) (layer "B.Cu") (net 3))
 (segment (start 36.768478 44.726173) (end 36.758968 44.741189) (width 0.25) (layer "B.Cu") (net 3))
 (segment (start 36.58323 42.963694) (end 36.603252 42.976373) (width 0.25) (layer "B.Cu") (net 3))
 (segment (start 36.82 44.54) (end 36.819563 44.557768) (width 0.25) (layer "B.Cu") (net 3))
 (segment (start 36.82 43.38) (end 36.819418 43.356307) (width 0.25) (layer "B.Cu") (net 3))
 (segment (start 36.748734 44.755721) (end 36.737798 44.769734) (width 0.25) (layer "B.Cu") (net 3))
 (segment (start 36.606172 44.888477) (end 36.621188 44.878968) (width 0.25) (layer "B.Cu") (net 3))
 (segment (start 36.810722 43.285801) (end 36.805529 43.262678) (width 0.25) (layer "B.Cu") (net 3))
 (segment (start 36.358691 42.895581) (end 36.382326 42.897325) (width 0.25) (layer "B.Cu") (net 3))
 (segment (start 36.83 43.52) (end 36.82 43.53) (width 0.25) (layer "B.Cu") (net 3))
 (segment (start 36.676065 44.833933) (end 36.713933 44.796066) (width 0.25) (layer "B.Cu") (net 3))
 (segment (start 36.622628 42.990019) (end 36.641311 43.0046) (width 0.25) (layer "B.Cu") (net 3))
 (segment (start 36.773641 43.173557) (end 36.762986 43.152388) (width 0.25) (layer "B.Cu") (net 3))
 (segment (start 36.762986 43.152388) (end 36.751305 43.131768) (width 0.25) (layer "B.Cu") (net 3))
 (segment (start 36.751305 43.131768) (end 36.738626 43.111746) (width 0.25) (layer "B.Cu") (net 3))
 (segment (start 36.79883 44.661998) (end 36.792433 44.678582) (width 0.25) (layer "B.Cu") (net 3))
 (segment (start 35.531357 42.468557) (end 35.542012 42.447389) (width 0.25) (layer "B.Cu") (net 4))
 (segment (start 35.697132 43.457132) (end 35.672619 43.431385) (width 0.25) (layer "B.Cu") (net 4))
 (segment (start 35.521753 42.490223) (end 35.531357 42.468557) (width 0.25) (layer "B.Cu") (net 4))
 (segment (start 35.6494 43.404468) (end 35.627529 43.376443) (width 0.25) (layer "B.Cu") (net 4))
 (segment (start 35.962673 42.152324) (end 35.939152 42.155225) (width 0.25) (layer "B.Cu") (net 4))
 (segment (start 35.540131 43.222163) (end 35.527337 43.188997) (width 0.25) (layer "B.Cu") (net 4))
 (segment (start 35.627529 43.376443) (end 35.60706 43.347379) (width 0.25) (layer "B.Cu") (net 4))
 (segment (start 36.893997 42.192337) (end 36.860242 42.181186) (width 0.25) (layer "B.Cu") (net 4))
 (segment (start 35.60706 43.347379) (end 35.588042 43.317346) (width 0.25) (layer "B.Cu") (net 4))
 (segment (start 35.72237 42.245018) (end 35.703687 42.259598) (width 0.25) (layer "B.Cu") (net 4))
 (segment (start 36.927163 42.205131) (end 36.893997 42.192337) (width 0.25) (layer "B.Cu") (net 4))
 (segment (start 35.554537 43.254662) (end 35.540131 43.222163) (width 0.25) (layer "B.Cu") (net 4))
 (segment (start 35.803557 42.196356) (end 35.782389 42.207012) (width 0.25) (layer "B.Cu") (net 4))
 (segment (start 36.685537 42.150872) (end 36.65 42.15) (width 0.25) (layer "B.Cu") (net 4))
 (segment (start 36.860242 42.181186) (end 36.825981 42.171705) (width 0.25) (layer "B.Cu") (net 4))
 (segment (start 35.542012 42.447389) (end 35.553694 42.426768) (width 0.25) (layer "B.Cu") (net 4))
 (segment (start 35.566373 42.406746) (end 35.580019 42.38737) (width 0.25) (layer "B.Cu") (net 4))
 (segment (start 35.485581 42.651307) (end 35.487324 42.627673) (width 0.25) (layer "B.Cu") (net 4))
 (segment (start 35.741746 42.231372) (end 35.72237 42.245018) (width 0.25) (layer "B.Cu") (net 4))
 (segment (start 36.01 42.15) (end 35.986308 42.15058) (width 0.25) (layer "B.Cu") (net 4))
 (segment (start 36.65 42.15) (end 36.01 42.15) (width 0.25) (layer "B.Cu") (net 4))
 (segment (start 35.488487 43.01599) (end 35.485872 42.980537) (width 0.25) (layer "B.Cu") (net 4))
 (segment (start 35.57052 43.286415) (end 35.554537 43.254662) (width 0.25) (layer "B.Cu") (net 4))
 (segment (start 35.610079 42.350741) (end 35.626421 42.333578) (width 0.25) (layer "B.Cu") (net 4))
 (segment (start 37.109468 42.3144) (end 37.081443 42.292529) (width 0.25) (layer "B.Cu") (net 4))
 (segment (start 36.756271 42.157839) (end 36.72099 42.153487) (width 0.25) (layer "B.Cu") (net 4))
 (segment (start 35.825223 42.186753) (end 35.803557 42.196356) (width 0.25) (layer "B.Cu") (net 4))
 (segment (start 35.516186 43.155242) (end 35.506705 43.120981) (width 0.25) (layer "B.Cu") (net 4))
 (segment (start 35.527337 43.188997) (end 35.516186 43.155242) (width 0.25) (layer "B.Cu") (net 4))
 (segment (start 35.498916 43.086296) (end 35.492839 43.051271) (width 0.25) (layer "B.Cu") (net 4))
 (segment (start 35.50579 42.534837) (end 35.513224 42.512334) (width 0.25) (layer "B.Cu") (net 4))
 (segment (start 36.959662 42.219537) (end 36.927163 42.205131) (width 0.25) (layer "B.Cu") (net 4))
 (segment (start 35.594599 42.368687) (end 35.610079 42.350741) (width 0.25) (layer "B.Cu") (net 4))
 (segment (start 37.052379 42.27206) (end 37.022346 42.253042) (width 0.25) (layer "B.Cu") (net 4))
 (segment (start 35.869837 42.17079) (end 35.847334 42.178224) (width 0.25) (layer "B.Cu") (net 4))
 (segment (start 35.782389 42.207012) (end 35.761768 42.218693) (width 0.25) (layer "B.Cu") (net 4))
 (segment (start 37.162132 42.362132) (end 37.136385 42.337619) (width 0.25) (layer "B.Cu") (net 4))
 (segment (start 37.162132 42.362132) (end 37.23 42.43) (width 0.25) (layer "B.Cu") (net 4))
 (segment (start 35.847334 42.178224) (end 35.825223 42.186753) (width 0.25) (layer "B.Cu") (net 4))
 (segment (start 36.791296 42.163916) (end 36.756271 42.157839) (width 0.25) (layer "B.Cu") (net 4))
 (segment (start 35.915801 42.159276) (end 35.892678 42.164469) (width 0.25) (layer "B.Cu") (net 4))
 (segment (start 35.490225 42.604152) (end 35.494277 42.580801) (width 0.25) (layer "B.Cu") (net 4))
 (segment (start 35.588042 43.317346) (end 35.57052 43.286415) (width 0.25) (layer "B.Cu") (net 4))
 (segment (start 36.72099 42.153487) (end 36.685537 42.150872) (width 0.25) (layer "B.Cu") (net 4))
 (segment (start 35.672619 43.431385) (end 35.6494 43.404468) (width 0.25) (layer "B.Cu") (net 4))
 (segment (start 36.825981 42.171705) (end 36.791296 42.163916) (width 0.25) (layer "B.Cu") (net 4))
 (segment (start 35.697132 43.457132) (end 36.13 43.89) (width 0.25) (layer "B.Cu") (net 4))
 (segment (start 35.553694 42.426768) (end 35.566373 42.406746) (width 0.25) (layer "B.Cu") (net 4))
 (segment (start 35.703687 42.259598) (end 35.685741 42.275078) (width 0.25) (layer "B.Cu") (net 4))
 (segment (start 35.685741 42.275078) (end 35.668578 42.29142) (width 0.25) (layer "B.Cu") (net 4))
 (segment (start 37.022346 42.253042) (end 36.991415 42.23552) (width 0.25) (layer "B.Cu") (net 4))
 (segment (start 35.485 42.675) (end 35.485 42.895) (width 0.25) (layer "B.Cu") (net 4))
 (segment (start 35.487324 42.627673) (end 35.490225 42.604152) (width 0.25) (layer "B.Cu") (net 4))
 (segment (start 35.485 42.945) (end 35.485 42.895) (width 0.25) (layer "B.Cu") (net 4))
 (segment (start 35.492839 43.051271) (end 35.488487 43.01599) (width 0.25) (layer "B.Cu") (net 4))
 (segment (start 35.485 42.675) (end 35.485581 42.651307) (width 0.25) (layer "B.Cu") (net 4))
 (segment (start 35.506705 43.120981) (end 35.498916 43.086296) (width 0.25) (layer "B.Cu") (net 4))
 (segment (start 35.668578 42.29142) (end 35.626421 42.333578) (width 0.25) (layer "B.Cu") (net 4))
 (segment (start 35.513224 42.512334) (end 35.521753 42.490223) (width 0.25) (layer "B.Cu") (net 4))
 (segment (start 35.892678 42.164469) (end 35.869837 42.17079) (width 0.25) (layer "B.Cu") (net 4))
 (segment (start 35.494277 42.580801) (end 35.499469 42.557678) (width 0.25) (layer "B.Cu") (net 4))
 (segment (start 36.991415 42.23552) (end 36.959662 42.219537) (width 0.25) (layer "B.Cu") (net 4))
 (segment (start 35.761768 42.218693) (end 35.741746 42.231372) (width 0.25) (layer "B.Cu") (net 4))
 (segment (start 37.136385 42.337619) (end 37.109468 42.3144) (width 0.25) (layer "B.Cu") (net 4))
 (segment (start 35.485872 42.980537) (end 35.485 42.945) (width 0.25) (layer "B.Cu") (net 4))
 (segment (start 35.986308 42.15058) (end 35.962673 42.152324) (width 0.25) (layer "B.Cu") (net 4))
 (segment (start 35.580019 42.38737) (end 35.594599 42.368687) (width 0.25) (layer "B.Cu") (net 4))
 (segment (start 35.939152 42.155225) (end 35.915801 42.159276) (width 0.25) (layer "B.Cu") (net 4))
 (segment (start 35.499469 42.557678) (end 35.50579 42.534837) (width 0.25) (layer "B.Cu") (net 4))
 (segment (start 37.081443 42.292529) (end 37.052379 42.27206) (width 0.25) (layer "B.Cu") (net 4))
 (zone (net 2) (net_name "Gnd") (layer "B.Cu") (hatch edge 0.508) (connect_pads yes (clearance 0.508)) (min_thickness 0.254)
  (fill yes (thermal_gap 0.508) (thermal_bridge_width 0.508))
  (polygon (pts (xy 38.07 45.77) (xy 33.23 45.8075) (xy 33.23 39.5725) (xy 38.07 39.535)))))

